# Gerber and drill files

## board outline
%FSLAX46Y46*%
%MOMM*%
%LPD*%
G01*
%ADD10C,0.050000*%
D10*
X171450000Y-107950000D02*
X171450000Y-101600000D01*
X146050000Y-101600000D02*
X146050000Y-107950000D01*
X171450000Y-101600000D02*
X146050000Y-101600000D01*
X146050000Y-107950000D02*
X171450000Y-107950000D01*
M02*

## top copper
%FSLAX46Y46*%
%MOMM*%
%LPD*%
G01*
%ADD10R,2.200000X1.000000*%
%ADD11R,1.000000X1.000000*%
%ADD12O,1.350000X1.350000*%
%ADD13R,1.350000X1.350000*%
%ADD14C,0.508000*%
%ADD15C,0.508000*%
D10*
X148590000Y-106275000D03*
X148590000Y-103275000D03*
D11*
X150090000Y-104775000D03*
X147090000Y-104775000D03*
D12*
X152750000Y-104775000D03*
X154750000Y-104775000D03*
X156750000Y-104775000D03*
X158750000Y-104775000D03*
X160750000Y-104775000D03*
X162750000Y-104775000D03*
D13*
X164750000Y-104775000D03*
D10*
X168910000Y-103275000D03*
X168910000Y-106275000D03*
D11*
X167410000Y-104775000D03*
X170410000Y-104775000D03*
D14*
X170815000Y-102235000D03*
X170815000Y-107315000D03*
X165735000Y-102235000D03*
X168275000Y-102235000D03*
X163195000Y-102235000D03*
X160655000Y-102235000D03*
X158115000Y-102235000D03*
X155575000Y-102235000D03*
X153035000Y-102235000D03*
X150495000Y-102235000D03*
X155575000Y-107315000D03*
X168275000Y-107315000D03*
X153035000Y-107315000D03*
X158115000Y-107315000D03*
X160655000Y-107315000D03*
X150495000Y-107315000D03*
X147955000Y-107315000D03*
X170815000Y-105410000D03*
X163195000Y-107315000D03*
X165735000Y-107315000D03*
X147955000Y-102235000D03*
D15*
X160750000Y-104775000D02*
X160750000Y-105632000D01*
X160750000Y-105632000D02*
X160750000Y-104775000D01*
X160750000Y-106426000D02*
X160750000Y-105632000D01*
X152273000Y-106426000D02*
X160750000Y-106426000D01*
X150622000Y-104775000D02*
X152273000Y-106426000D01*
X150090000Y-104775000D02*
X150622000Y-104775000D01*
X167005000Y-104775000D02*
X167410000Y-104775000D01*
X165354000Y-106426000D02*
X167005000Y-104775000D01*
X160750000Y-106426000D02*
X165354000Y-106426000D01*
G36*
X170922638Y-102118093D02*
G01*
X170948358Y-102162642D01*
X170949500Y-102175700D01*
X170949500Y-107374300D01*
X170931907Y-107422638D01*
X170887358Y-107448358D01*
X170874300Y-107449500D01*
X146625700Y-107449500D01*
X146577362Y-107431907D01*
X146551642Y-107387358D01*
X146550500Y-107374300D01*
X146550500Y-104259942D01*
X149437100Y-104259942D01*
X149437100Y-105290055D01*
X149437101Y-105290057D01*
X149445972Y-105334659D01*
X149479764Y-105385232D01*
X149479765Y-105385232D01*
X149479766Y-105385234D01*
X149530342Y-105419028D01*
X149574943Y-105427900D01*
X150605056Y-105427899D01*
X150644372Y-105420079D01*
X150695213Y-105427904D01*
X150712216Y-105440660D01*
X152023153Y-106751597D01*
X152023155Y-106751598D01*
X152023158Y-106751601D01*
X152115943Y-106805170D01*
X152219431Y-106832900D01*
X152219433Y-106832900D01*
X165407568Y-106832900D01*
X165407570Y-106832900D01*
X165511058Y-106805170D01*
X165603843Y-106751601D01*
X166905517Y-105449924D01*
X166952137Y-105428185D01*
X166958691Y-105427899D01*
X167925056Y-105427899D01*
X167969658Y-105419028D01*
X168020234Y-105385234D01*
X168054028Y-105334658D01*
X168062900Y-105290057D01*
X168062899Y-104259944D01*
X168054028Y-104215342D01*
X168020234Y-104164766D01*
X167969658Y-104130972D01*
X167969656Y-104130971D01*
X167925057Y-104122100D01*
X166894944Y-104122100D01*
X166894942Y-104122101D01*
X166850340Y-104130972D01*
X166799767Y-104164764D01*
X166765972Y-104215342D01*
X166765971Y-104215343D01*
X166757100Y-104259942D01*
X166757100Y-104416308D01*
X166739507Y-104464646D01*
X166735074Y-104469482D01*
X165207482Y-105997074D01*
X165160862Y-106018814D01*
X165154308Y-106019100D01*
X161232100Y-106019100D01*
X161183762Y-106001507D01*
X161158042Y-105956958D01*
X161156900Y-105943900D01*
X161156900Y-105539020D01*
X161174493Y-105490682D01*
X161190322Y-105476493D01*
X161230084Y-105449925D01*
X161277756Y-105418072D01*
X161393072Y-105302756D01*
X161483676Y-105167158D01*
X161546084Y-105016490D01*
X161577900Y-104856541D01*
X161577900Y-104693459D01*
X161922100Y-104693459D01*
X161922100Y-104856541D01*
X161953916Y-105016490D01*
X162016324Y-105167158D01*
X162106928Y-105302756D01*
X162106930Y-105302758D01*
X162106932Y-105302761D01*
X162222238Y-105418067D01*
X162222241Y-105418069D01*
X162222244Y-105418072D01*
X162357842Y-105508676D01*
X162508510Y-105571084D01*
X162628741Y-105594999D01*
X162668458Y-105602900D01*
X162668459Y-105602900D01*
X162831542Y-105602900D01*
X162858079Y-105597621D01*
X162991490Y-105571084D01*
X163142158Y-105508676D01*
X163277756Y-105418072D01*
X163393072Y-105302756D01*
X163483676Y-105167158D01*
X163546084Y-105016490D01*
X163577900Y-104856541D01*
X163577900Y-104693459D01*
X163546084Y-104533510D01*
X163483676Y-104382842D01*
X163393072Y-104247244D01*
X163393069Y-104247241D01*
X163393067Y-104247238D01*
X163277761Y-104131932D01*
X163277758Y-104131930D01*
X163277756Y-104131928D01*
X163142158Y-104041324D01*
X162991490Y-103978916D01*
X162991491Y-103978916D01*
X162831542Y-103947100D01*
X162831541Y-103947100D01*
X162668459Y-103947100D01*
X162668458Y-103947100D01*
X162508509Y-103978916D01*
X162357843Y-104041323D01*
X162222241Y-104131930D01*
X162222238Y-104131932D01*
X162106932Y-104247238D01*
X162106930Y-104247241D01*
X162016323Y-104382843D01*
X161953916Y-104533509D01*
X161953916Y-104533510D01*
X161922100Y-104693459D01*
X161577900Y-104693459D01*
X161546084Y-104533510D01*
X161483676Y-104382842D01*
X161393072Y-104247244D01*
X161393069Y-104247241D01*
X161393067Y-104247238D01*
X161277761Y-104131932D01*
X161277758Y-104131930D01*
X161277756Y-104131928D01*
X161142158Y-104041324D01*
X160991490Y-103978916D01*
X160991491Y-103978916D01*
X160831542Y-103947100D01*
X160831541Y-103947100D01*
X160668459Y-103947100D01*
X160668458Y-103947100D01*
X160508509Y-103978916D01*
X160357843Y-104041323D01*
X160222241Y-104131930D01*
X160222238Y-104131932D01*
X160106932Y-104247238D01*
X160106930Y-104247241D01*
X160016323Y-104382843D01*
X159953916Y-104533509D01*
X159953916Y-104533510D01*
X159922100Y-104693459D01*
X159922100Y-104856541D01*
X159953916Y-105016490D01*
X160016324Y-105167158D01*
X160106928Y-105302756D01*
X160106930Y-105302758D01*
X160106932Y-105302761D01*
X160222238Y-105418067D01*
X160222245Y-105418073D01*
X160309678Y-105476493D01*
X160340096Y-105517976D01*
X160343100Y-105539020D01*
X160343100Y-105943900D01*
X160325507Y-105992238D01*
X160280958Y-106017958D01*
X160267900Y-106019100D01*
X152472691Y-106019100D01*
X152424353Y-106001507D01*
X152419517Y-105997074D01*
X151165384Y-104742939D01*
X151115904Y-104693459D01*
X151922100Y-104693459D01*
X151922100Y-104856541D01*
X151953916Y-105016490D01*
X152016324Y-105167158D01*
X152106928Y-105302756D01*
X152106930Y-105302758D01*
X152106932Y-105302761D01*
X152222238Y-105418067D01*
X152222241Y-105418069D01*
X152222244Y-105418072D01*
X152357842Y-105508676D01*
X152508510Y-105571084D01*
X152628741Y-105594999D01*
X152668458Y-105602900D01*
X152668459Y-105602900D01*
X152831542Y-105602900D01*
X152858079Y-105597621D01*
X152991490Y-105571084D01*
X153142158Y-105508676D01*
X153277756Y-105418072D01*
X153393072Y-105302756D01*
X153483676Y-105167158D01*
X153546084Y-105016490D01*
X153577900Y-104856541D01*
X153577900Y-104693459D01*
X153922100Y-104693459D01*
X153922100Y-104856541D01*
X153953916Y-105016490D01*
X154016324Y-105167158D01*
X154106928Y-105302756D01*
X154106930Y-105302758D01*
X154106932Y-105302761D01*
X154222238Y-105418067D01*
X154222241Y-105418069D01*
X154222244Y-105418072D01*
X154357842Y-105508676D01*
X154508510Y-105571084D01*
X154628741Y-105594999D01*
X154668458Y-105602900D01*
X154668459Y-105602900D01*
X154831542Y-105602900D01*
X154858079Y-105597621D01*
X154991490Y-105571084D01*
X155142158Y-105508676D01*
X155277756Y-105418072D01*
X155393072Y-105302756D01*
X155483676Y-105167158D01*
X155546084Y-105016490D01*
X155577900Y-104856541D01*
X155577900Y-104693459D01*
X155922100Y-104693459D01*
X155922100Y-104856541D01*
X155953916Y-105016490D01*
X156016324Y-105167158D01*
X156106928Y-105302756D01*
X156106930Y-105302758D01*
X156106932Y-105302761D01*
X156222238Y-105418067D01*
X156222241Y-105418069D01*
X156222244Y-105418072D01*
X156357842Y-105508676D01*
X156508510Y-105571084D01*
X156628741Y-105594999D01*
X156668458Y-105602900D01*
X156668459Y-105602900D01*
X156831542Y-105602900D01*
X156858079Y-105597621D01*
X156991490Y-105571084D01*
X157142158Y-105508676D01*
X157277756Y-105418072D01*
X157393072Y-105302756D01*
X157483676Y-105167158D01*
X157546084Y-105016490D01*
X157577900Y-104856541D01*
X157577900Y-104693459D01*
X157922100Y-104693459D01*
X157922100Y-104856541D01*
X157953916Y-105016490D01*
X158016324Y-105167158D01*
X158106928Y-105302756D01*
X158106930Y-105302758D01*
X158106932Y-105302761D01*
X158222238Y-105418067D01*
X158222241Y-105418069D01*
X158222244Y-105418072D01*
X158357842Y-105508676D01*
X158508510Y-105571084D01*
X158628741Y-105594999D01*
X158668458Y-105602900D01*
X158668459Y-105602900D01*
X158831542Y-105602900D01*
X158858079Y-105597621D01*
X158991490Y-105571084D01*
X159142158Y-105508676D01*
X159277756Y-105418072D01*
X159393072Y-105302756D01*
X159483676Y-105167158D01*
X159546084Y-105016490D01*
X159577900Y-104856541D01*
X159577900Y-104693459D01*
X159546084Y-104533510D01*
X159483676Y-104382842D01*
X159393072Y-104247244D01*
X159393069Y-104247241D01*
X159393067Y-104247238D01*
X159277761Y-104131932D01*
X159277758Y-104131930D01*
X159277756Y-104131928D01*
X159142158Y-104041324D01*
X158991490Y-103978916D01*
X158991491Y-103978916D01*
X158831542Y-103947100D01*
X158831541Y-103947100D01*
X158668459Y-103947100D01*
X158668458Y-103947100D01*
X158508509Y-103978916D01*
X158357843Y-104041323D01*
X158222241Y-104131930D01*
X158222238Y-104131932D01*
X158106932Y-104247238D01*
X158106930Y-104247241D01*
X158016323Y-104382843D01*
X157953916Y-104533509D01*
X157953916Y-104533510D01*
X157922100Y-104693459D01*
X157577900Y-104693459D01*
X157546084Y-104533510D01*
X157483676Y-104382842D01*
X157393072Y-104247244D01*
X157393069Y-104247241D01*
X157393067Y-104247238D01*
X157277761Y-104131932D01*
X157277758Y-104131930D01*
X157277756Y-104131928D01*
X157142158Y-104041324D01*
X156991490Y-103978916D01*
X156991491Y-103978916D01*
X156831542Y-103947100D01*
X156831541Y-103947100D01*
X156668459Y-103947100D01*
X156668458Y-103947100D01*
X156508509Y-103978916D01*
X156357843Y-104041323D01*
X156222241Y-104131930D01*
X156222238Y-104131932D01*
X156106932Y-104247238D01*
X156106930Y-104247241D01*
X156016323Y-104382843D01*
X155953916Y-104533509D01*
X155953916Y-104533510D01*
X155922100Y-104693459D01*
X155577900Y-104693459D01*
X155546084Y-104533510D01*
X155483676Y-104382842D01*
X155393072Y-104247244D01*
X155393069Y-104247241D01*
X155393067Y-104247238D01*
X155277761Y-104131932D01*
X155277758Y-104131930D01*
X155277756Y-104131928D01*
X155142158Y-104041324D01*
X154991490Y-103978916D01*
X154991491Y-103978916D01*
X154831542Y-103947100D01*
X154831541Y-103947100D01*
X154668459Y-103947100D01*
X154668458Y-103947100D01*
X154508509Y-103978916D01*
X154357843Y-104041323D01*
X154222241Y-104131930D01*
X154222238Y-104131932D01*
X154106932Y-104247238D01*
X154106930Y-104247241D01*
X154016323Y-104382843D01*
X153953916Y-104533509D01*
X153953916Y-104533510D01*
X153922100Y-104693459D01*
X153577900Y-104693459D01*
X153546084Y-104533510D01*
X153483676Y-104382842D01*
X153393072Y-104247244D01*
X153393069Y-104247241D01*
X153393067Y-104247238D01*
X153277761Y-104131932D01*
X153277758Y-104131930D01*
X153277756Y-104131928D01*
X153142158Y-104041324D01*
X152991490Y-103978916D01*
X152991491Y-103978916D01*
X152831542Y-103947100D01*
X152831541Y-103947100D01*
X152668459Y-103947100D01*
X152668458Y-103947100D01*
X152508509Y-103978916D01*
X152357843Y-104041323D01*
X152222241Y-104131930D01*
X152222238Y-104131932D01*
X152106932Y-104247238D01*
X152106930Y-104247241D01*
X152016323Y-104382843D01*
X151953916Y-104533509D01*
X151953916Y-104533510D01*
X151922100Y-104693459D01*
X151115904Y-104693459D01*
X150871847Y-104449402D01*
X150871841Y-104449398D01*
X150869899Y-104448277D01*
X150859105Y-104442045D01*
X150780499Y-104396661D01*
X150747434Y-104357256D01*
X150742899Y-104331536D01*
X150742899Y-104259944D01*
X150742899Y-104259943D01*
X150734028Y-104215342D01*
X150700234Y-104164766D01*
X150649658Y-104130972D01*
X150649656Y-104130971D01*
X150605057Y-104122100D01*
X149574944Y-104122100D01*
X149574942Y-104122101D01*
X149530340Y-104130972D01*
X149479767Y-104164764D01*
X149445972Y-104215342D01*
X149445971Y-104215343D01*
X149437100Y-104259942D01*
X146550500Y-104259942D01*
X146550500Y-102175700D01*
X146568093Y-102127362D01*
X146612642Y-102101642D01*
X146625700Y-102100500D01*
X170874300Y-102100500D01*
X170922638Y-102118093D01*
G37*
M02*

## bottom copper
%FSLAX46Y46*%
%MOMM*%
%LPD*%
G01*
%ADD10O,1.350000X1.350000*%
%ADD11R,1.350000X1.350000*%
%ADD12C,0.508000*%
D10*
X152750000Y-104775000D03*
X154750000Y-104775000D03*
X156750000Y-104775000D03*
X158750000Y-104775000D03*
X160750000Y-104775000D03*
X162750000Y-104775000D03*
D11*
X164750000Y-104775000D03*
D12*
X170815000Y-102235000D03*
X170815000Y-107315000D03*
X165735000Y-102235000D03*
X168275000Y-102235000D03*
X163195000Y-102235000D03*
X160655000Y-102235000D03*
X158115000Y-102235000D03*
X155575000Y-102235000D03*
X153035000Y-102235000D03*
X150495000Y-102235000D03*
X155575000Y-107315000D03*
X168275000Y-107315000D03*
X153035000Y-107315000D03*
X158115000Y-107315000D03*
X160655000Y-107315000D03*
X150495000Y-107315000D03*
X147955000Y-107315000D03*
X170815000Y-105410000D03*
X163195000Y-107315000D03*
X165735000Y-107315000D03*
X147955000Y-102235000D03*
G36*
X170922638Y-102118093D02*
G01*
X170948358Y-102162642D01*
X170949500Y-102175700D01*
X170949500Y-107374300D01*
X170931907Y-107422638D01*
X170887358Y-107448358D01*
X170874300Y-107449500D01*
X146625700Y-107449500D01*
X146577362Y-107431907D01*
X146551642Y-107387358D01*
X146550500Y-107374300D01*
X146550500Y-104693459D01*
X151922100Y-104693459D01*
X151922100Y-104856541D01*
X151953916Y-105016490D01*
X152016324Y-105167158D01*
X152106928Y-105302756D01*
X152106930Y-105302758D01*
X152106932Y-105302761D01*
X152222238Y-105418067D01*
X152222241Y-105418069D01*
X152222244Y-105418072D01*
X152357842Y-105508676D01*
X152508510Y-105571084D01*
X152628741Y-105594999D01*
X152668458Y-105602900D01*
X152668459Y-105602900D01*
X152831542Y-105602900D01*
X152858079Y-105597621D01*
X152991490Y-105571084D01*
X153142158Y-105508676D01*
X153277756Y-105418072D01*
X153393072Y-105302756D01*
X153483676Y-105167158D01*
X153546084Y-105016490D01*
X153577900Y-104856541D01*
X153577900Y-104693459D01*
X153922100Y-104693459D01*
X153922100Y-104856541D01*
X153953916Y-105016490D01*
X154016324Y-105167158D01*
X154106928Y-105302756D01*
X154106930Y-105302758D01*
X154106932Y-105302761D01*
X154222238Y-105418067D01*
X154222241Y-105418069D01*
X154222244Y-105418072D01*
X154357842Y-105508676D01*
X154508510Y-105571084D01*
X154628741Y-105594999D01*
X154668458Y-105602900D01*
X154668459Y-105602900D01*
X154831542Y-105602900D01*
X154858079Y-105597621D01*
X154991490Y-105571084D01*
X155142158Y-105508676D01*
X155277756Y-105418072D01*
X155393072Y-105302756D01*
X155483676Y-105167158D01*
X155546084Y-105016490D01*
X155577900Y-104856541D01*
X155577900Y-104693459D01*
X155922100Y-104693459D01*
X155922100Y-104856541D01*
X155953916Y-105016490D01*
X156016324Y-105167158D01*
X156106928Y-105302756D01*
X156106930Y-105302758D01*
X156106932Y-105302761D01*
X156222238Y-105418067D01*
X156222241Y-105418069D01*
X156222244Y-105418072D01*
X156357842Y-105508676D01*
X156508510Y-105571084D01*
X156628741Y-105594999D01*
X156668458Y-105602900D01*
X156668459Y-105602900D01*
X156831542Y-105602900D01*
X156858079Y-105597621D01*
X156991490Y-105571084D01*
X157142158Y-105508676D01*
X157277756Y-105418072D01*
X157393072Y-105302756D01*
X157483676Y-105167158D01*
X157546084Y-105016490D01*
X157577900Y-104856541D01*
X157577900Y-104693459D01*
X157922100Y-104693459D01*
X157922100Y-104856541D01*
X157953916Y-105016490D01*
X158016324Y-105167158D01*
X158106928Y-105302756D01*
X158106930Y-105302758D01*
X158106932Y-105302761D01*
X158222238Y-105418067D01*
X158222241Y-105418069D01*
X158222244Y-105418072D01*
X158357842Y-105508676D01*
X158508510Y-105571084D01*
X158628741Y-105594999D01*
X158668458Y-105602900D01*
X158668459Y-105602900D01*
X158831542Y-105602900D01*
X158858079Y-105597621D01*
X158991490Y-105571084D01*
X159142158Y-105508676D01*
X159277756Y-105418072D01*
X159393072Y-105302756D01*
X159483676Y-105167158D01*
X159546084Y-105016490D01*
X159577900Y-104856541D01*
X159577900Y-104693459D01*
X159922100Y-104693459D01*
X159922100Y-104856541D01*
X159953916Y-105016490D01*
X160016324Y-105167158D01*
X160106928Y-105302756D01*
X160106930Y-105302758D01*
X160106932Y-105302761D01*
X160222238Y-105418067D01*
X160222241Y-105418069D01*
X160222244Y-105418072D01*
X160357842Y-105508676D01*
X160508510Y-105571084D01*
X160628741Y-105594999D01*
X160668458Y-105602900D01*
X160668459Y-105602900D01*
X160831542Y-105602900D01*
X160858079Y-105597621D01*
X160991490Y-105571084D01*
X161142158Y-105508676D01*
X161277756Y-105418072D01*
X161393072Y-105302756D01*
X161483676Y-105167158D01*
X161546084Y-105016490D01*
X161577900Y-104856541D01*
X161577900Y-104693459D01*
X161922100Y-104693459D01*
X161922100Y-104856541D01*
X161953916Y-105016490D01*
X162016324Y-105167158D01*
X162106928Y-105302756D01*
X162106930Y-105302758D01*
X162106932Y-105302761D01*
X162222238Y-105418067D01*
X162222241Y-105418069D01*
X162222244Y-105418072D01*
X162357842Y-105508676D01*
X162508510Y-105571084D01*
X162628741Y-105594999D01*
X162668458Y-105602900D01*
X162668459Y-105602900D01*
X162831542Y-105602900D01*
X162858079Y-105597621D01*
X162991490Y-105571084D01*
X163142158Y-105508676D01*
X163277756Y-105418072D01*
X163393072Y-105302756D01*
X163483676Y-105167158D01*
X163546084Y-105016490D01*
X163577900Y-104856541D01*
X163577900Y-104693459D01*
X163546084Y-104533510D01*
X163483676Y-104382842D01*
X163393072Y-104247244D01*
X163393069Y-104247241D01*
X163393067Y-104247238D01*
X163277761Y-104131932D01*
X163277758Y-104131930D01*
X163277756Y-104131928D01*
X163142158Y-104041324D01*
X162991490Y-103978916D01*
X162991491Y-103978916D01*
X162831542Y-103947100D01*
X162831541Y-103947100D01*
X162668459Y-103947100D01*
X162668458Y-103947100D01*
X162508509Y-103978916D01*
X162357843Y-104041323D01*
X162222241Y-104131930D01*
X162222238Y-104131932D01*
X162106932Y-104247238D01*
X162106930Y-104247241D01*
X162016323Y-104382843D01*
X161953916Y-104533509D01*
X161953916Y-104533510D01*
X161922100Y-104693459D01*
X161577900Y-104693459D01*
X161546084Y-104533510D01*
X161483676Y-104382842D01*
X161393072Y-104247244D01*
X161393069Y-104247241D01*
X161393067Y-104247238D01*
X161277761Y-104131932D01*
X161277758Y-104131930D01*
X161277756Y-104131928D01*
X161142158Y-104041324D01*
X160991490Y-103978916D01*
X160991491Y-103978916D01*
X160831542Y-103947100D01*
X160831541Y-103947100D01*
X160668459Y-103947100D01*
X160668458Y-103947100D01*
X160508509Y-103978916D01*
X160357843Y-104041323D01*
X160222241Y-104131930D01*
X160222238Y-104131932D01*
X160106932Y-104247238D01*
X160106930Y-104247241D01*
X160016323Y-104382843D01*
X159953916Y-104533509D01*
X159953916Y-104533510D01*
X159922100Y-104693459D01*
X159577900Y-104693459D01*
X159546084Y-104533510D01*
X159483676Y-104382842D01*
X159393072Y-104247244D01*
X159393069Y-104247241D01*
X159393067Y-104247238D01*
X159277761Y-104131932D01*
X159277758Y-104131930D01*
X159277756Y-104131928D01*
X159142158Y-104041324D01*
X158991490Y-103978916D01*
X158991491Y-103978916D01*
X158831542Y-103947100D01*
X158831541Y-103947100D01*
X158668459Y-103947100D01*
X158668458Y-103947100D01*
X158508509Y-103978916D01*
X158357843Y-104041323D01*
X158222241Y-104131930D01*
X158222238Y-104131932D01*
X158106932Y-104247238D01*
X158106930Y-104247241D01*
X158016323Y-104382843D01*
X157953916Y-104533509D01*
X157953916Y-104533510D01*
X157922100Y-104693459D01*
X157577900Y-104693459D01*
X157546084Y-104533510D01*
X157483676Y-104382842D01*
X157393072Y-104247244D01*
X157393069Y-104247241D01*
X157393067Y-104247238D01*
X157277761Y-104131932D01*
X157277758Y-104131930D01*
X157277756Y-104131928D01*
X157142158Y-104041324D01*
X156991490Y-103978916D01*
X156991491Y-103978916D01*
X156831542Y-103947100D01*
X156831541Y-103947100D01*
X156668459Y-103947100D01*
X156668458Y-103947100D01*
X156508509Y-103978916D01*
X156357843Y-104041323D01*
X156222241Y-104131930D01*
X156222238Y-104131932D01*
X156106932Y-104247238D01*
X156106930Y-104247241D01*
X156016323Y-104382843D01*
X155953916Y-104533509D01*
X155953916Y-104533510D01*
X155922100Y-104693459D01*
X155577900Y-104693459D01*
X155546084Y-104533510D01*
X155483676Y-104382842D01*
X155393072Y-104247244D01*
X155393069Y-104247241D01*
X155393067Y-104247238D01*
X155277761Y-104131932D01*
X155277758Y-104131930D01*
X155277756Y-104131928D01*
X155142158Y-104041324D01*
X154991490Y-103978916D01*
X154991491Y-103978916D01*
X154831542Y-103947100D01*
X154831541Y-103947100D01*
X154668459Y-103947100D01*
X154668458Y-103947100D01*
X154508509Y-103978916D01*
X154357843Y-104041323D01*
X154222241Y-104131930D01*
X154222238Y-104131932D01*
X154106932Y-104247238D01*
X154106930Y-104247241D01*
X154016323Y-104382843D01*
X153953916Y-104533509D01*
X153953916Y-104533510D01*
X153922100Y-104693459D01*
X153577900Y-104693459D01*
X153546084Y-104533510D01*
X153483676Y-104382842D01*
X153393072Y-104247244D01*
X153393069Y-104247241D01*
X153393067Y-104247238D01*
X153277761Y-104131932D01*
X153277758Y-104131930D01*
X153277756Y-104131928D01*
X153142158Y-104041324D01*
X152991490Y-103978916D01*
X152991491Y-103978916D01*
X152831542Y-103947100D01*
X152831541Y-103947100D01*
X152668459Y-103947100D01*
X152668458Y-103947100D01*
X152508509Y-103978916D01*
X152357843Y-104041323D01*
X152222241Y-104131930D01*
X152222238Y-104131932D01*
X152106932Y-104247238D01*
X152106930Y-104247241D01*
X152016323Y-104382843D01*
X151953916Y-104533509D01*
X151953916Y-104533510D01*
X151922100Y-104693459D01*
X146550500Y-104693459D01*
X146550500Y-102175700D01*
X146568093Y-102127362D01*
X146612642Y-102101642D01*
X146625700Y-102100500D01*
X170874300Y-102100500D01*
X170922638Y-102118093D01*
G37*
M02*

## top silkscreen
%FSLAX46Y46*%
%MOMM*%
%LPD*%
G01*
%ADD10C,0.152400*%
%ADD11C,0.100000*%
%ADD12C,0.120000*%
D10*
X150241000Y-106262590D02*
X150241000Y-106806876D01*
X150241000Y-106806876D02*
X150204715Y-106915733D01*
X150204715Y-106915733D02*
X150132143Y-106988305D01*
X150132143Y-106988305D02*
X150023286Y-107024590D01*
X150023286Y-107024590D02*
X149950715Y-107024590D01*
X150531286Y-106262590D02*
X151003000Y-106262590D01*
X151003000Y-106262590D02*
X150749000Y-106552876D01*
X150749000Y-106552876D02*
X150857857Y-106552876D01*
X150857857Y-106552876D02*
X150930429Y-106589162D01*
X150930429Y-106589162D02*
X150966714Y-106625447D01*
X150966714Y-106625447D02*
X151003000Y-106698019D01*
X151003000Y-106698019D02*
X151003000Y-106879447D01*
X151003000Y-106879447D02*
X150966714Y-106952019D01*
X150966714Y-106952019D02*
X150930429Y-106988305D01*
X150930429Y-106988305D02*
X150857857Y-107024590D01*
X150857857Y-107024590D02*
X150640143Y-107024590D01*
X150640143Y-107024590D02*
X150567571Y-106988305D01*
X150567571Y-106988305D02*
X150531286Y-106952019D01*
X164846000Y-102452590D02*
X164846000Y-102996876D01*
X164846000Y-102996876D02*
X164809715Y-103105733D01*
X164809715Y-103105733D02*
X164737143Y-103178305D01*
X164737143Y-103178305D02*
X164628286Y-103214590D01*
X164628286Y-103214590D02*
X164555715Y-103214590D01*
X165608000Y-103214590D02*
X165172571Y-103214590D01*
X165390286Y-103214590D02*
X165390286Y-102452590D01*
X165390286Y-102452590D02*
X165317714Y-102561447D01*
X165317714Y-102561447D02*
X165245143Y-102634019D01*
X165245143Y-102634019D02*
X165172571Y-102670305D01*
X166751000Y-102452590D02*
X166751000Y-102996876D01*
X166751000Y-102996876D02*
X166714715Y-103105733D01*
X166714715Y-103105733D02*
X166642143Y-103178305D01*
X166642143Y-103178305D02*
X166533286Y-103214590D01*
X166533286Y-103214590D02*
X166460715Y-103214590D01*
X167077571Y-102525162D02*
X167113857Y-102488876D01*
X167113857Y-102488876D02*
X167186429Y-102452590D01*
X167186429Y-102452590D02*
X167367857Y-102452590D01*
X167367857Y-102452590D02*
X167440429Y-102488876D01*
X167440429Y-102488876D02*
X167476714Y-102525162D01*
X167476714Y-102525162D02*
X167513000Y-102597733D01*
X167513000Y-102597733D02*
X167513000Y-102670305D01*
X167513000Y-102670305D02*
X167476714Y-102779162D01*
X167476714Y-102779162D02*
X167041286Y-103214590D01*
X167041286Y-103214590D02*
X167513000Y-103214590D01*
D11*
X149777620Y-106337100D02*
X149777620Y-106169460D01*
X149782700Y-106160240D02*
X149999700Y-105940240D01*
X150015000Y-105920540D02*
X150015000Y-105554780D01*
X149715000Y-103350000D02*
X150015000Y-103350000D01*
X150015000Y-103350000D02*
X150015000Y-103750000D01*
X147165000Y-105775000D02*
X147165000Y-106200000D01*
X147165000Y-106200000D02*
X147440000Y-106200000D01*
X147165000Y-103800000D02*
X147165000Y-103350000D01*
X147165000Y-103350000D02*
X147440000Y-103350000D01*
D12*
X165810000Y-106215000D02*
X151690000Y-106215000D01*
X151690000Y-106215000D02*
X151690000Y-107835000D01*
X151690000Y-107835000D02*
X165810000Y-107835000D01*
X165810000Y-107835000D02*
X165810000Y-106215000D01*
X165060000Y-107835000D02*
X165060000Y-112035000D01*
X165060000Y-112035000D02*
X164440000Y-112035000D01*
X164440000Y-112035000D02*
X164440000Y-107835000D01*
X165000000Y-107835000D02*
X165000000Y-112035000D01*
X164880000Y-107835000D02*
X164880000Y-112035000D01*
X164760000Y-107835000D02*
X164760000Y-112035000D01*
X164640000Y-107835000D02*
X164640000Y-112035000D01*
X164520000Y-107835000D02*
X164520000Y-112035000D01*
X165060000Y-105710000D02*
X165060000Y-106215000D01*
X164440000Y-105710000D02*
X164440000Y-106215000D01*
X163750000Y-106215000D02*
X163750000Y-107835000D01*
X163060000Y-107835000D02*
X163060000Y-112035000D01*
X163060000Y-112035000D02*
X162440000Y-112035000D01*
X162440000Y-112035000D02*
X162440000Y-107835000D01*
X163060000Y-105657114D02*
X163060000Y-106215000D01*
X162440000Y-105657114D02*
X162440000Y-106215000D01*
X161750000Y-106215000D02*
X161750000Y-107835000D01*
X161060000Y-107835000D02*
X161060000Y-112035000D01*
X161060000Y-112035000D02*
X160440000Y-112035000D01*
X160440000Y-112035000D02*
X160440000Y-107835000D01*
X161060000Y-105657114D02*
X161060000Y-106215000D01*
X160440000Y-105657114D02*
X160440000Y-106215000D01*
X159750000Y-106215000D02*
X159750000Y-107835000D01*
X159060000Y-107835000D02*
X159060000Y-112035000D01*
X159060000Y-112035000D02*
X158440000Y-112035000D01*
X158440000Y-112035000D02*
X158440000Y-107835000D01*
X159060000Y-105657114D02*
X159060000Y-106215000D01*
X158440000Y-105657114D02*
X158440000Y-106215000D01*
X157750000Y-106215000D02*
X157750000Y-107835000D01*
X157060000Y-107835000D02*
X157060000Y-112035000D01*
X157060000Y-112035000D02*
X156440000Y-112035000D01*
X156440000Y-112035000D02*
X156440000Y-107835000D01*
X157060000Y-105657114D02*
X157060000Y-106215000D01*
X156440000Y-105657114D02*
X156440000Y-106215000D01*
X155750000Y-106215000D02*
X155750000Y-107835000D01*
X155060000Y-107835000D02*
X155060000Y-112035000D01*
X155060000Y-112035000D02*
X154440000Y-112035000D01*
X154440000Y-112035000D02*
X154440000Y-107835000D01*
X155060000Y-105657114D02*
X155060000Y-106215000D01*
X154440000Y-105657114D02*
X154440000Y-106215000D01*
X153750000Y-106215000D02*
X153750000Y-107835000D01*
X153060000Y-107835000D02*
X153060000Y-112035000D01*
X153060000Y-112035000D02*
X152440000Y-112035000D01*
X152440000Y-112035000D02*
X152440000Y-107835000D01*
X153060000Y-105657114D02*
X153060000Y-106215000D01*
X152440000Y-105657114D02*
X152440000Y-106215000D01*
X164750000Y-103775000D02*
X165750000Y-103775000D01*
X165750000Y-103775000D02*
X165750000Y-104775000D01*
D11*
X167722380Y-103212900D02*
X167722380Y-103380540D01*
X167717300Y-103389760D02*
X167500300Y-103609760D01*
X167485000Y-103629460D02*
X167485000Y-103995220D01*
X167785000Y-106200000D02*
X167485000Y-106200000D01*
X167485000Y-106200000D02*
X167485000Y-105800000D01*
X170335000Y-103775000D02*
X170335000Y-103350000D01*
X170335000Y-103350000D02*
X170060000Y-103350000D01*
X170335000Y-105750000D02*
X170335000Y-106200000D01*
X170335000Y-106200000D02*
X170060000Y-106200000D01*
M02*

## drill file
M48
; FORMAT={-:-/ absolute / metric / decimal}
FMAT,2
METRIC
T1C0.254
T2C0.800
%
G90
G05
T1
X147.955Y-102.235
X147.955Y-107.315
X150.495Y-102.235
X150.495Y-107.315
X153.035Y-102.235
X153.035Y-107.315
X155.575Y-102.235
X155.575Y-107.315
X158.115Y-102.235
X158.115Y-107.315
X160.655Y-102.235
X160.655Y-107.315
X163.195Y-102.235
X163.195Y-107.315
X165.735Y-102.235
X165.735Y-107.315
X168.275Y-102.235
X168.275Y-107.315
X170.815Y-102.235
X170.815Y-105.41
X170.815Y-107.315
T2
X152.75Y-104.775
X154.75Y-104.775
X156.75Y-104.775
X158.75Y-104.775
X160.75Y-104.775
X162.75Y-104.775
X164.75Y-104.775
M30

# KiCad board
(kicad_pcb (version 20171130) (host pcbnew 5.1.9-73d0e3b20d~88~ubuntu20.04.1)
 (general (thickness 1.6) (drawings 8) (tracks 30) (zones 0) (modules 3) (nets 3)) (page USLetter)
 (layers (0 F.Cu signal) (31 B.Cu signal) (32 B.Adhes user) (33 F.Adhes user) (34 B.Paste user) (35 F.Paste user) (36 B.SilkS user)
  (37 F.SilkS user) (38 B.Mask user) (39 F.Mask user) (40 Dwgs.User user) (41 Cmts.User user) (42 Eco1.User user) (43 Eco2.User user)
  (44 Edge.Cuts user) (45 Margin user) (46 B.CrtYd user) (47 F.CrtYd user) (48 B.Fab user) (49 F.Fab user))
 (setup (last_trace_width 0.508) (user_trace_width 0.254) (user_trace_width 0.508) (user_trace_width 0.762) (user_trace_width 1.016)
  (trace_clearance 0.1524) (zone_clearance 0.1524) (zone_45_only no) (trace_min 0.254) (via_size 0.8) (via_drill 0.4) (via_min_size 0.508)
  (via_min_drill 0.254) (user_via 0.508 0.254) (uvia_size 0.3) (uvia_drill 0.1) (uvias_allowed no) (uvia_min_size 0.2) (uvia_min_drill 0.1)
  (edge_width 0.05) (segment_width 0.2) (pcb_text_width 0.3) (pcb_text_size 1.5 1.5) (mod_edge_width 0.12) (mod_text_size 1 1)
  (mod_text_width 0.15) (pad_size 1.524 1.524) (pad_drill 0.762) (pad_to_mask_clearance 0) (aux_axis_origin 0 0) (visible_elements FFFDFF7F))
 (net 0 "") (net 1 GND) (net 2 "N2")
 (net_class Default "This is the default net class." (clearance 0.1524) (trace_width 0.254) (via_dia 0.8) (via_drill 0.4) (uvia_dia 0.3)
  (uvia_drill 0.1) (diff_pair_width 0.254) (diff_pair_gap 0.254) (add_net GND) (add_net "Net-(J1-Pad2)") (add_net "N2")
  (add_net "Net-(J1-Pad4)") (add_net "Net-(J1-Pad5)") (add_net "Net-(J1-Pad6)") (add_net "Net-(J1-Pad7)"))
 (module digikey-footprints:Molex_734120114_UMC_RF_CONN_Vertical (layer F.Cu) (at 148.59 104.775 90)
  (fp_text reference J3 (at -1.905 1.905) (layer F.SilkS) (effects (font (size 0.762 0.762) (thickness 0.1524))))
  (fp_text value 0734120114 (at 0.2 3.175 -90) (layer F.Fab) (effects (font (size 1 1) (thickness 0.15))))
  (fp_line (start -1.5621 1.18762) (end -1.39446 1.18762) (layer F.SilkS) (width 0.1))
  (fp_line (start -1.38524 1.1927) (end -1.16524 1.4097) (layer F.SilkS) (width 0.1))
  (fp_line (start -1.14554 1.425) (end -0.77978 1.425) (layer F.SilkS) (width 0.1))
  (fp_line (start 1.425 1.125) (end 1.425 1.425) (layer F.SilkS) (width 0.1))
  (fp_line (start 1.425 1.425) (end 1.025 1.425) (layer F.SilkS) (width 0.1))
  (fp_line (start -1 -1.425) (end -1.425 -1.425) (layer F.SilkS) (width 0.1))
  (fp_line (start -1.425 -1.425) (end -1.425 -1.15) (layer F.SilkS) (width 0.1))
  (fp_line (start 0.975 -1.425) (end 1.425 -1.425) (layer F.SilkS) (width 0.1))
  (fp_line (start 1.425 -1.425) (end 1.425 -1.15) (layer F.SilkS) (width 0.1))
  (pad 1 smd rect (at -1.5 0 90) (size 1 2.2) (layers F.Cu F.Paste F.Mask) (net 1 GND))
  (pad 1 smd rect (at 1.5 0 90) (size 1 2.2) (layers F.Cu F.Paste F.Mask) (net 1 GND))
  (pad 2 smd rect (at 0 1.5 90) (size 1 1) (layers F.Cu F.Paste F.Mask) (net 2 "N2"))
  (pad 1 smd rect (at 0 -1.5 90) (size 1 1) (layers F.Cu F.Paste F.Mask) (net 1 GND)))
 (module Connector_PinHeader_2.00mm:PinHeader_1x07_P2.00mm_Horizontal (layer F.Cu) (at 164.75 104.775 270)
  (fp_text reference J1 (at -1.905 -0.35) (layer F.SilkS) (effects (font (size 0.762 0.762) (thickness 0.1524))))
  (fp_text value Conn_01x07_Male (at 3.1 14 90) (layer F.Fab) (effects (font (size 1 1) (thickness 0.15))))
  (fp_line (start 1.44 -1.06) (end 1.44 13.06) (layer F.SilkS) (width 0.12))
  (fp_line (start 1.44 13.06) (end 3.06 13.06) (layer F.SilkS) (width 0.12))
  (fp_line (start 3.06 13.06) (end 3.06 -1.06) (layer F.SilkS) (width 0.12))
  (fp_line (start 3.06 -1.06) (end 1.44 -1.06) (layer F.SilkS) (width 0.12))
  (fp_line (start 3.06 -0.31) (end 7.26 -0.31) (layer F.SilkS) (width 0.12))
  (fp_line (start 7.26 -0.31) (end 7.26 0.31) (layer F.SilkS) (width 0.12))
  (fp_line (start 7.26 0.31) (end 3.06 0.31) (layer F.SilkS) (width 0.12))
  (fp_line (start 3.06 -0.25) (end 7.26 -0.25) (layer F.SilkS) (width 0.12))
  (fp_line (start 3.06 -0.13) (end 7.26 -0.13) (layer F.SilkS) (width 0.12))
  (fp_line (start 3.06 -0.01) (end 7.26 -0.01) (layer F.SilkS) (width 0.12))
  (fp_line (start 3.06 0.11) (end 7.26 0.11) (layer F.SilkS) (width 0.12))
  (fp_line (start 3.06 0.23) (end 7.26 0.23) (layer F.SilkS) (width 0.12))
  (fp_line (start 0.935 -0.31) (end 1.44 -0.31) (layer F.SilkS) (width 0.12))
  (fp_line (start 0.935 0.31) (end 1.44 0.31) (layer F.SilkS) (width 0.12))
  (fp_line (start 1.44 1) (end 3.06 1) (layer F.SilkS) (width 0.12))
  (fp_line (start 3.06 1.69) (end 7.26 1.69) (layer F.SilkS) (width 0.12))
  (fp_line (start 7.26 1.69) (end 7.26 2.31) (layer F.SilkS) (width 0.12))
  (fp_line (start 7.26 2.31) (end 3.06 2.31) (layer F.SilkS) (width 0.12))
  (fp_line (start 0.882114 1.69) (end 1.44 1.69) (layer F.SilkS) (width 0.12))
  (fp_line (start 0.882114 2.31) (end 1.44 2.31) (layer F.SilkS) (width 0.12))
  (fp_line (start 1.44 3) (end 3.06 3) (layer F.SilkS) (width 0.12))
  (fp_line (start 3.06 3.69) (end 7.26 3.69) (layer F.SilkS) (width 0.12))
  (fp_line (start 7.26 3.69) (end 7.26 4.31) (layer F.SilkS) (width 0.12))
  (fp_line (start 7.26 4.31) (end 3.06 4.31) (layer F.SilkS) (width 0.12))
  (fp_line (start 0.882114 3.69) (end 1.44 3.69) (layer F.SilkS) (width 0.12))
  (fp_line (start 0.882114 4.31) (end 1.44 4.31) (layer F.SilkS) (width 0.12))
  (fp_line (start 1.44 5) (end 3.06 5) (layer F.SilkS) (width 0.12))
  (fp_line (start 3.06 5.69) (end 7.26 5.69) (layer F.SilkS) (width 0.12))
  (fp_line (start 7.26 5.69) (end 7.26 6.31) (layer F.SilkS) (width 0.12))
  (fp_line (start 7.26 6.31) (end 3.06 6.31) (layer F.SilkS) (width 0.12))
  (fp_line (start 0.882114 5.69) (end 1.44 5.69) (layer F.SilkS) (width 0.12))
  (fp_line (start 0.882114 6.31) (end 1.44 6.31) (layer F.SilkS) (width 0.12))
  (fp_line (start 1.44 7) (end 3.06 7) (layer F.SilkS) (width 0.12))
  (fp_line (start 3.06 7.69) (end 7.26 7.69) (layer F.SilkS) (width 0.12))
  (fp_line (start 7.26 7.69) (end 7.26 8.31) (layer F.SilkS) (width 0.12))
  (fp_line (start 7.26 8.31) (end 3.06 8.31) (layer F.SilkS) (width 0.12))
  (fp_line (start 0.882114 7.69) (end 1.44 7.69) (layer F.SilkS) (width 0.12))
  (fp_line (start 0.882114 8.31) (end 1.44 8.31) (layer F.SilkS) (width 0.12))
  (fp_line (start 1.44 9) (end 3.06 9) (layer F.SilkS) (width 0.12))
  (fp_line (start 3.06 9.69) (end 7.26 9.69) (layer F.SilkS) (width 0.12))
  (fp_line (start 7.26 9.69) (end 7.26 10.31) (layer F.SilkS) (width 0.12))
  (fp_line (start 7.26 10.31) (end 3.06 10.31) (layer F.SilkS) (width 0.12))
  (fp_line (start 0.882114 9.69) (end 1.44 9.69) (layer F.SilkS) (width 0.12))
  (fp_line (start 0.882114 10.31) (end 1.44 10.31) (layer F.SilkS) (width 0.12))
  (fp_line (start 1.44 11) (end 3.06 11) (layer F.SilkS) (width 0.12))
  (fp_line (start 3.06 11.69) (end 7.26 11.69) (layer F.SilkS) (width 0.12))
  (fp_line (start 7.26 11.69) (end 7.26 12.31) (layer F.SilkS) (width 0.12))
  (fp_line (start 7.26 12.31) (end 3.06 12.31) (layer F.SilkS) (width 0.12))
  (fp_line (start 0.882114 11.69) (end 1.44 11.69) (layer F.SilkS) (width 0.12))
  (fp_line (start 0.882114 12.31) (end 1.44 12.31) (layer F.SilkS) (width 0.12))
  (fp_line (start -1 0) (end -1 -1) (layer F.SilkS) (width 0.12))
  (fp_line (start -1 -1) (end 0 -1) (layer F.SilkS) (width 0.12))
  (pad 7 thru_hole oval (at 0 12 270) (size 1.35 1.35) (drill 0.8) (layers *.Cu *.Mask))
  (pad 6 thru_hole oval (at 0 10 270) (size 1.35 1.35) (drill 0.8) (layers *.Cu *.Mask))
  (pad 5 thru_hole oval (at 0 8 270) (size 1.35 1.35) (drill 0.8) (layers *.Cu *.Mask))
  (pad 4 thru_hole oval (at 0 6 270) (size 1.35 1.35) (drill 0.8) (layers *.Cu *.Mask))
  (pad 3 thru_hole oval (at 0 4 270) (size 1.35 1.35) (drill 0.8) (layers *.Cu *.Mask) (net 2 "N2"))
  (pad 2 thru_hole oval (at 0 2 270) (size 1.35 1.35) (drill 0.8) (layers *.Cu *.Mask))
  (pad 1 thru_hole rect (at 0 0 270) (size 1.35 1.35) (drill 0.8) (layers *.Cu *.Mask) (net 1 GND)))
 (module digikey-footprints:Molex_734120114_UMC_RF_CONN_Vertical (layer F.Cu) (at 168.91 104.775 270)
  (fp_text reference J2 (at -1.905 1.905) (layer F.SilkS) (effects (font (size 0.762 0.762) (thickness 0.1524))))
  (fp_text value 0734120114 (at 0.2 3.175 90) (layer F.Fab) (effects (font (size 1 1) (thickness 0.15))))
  (fp_line (start -1.5621 1.18762) (end -1.39446 1.18762) (layer F.SilkS) (width 0.1))
  (fp_line (start -1.38524 1.1927) (end -1.16524 1.4097) (layer F.SilkS) (width 0.1))
  (fp_line (start -1.14554 1.425) (end -0.77978 1.425) (layer F.SilkS) (width 0.1))
  (fp_line (start 1.425 1.125) (end 1.425 1.425) (layer F.SilkS) (width 0.1))
  (fp_line (start 1.425 1.425) (end 1.025 1.425) (layer F.SilkS) (width 0.1))
  (fp_line (start -1 -1.425) (end -1.425 -1.425) (layer F.SilkS) (width 0.1))
  (fp_line (start -1.425 -1.425) (end -1.425 -1.15) (layer F.SilkS) (width 0.1))
  (fp_line (start 0.975 -1.425) (end 1.425 -1.425) (layer F.SilkS) (width 0.1))
  (fp_line (start 1.425 -1.425) (end 1.425 -1.15) (layer F.SilkS) (width 0.1))
  (pad 1 smd rect (at -1.5 0 270) (size 1 2.2) (layers F.Cu F.Paste F.Mask) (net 1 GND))
  (pad 1 smd rect (at 1.5 0 270) (size 1 2.2) (layers F.Cu F.Paste F.Mask) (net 1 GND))
  (pad 2 smd rect (at 0 1.5 270) (size 1 1) (layers F.Cu F.Paste F.Mask) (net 2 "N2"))
  (pad 1 smd rect (at 0 -1.5 270) (size 1 1) (layers F.Cu F.Paste F.Mask) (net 1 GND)))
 (gr_line (start 171.45 107.95) (end 171.45 101.6) (layer Edge.Cuts) (width 0.05))
 (gr_line (start 146.05 101.6) (end 146.05 107.95) (layer Edge.Cuts) (width 0.05))
 (gr_line (start 171.45 101.6) (end 146.05 101.6) (layer Edge.Cuts) (width 0.05))
 (gr_line (start 146.05 107.95) (end 171.45 107.95) (layer Edge.Cuts) (width 0.05))
 (segment (start 160.75 104.775) (end 160.75 105.632) (width 0.508) (layer F.Cu) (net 2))
 (segment (start 160.75 105.632) (end 160.75 104.775) (width 0.508) (layer F.Cu) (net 2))
 (segment (start 160.75 106.426) (end 160.75 105.632) (width 0.508) (layer F.Cu) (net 2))
 (segment (start 152.273 106.426) (end 160.75 106.426) (width 0.508) (layer F.Cu) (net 2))
 (segment (start 150.622 104.775) (end 152.273 106.426) (width 0.508) (layer F.Cu) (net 2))
 (segment (start 150.09 104.775) (end 150.622 104.775) (width 0.508) (layer F.Cu) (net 2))
 (segment (start 167.005 104.775) (end 167.41 104.775) (width 0.508) (layer F.Cu) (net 2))
 (segment (start 165.354 106.426) (end 167.005 104.775) (width 0.508) (layer F.Cu) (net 2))
 (segment (start 160.75 106.426) (end 165.354 106.426) (width 0.508) (layer F.Cu) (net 2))
 (via (at 170.815 102.235) (size 0.508) (drill 0.254) (layers F.Cu B.Cu) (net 1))
 (via (at 170.815 107.315) (size 0.508) (drill 0.254) (layers F.Cu B.Cu) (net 1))
 (via (at 165.735 102.235) (size 0.508) (drill 0.254) (layers F.Cu B.Cu) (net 1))
 (via (at 168.275 102.235) (size 0.508) (drill 0.254) (layers F.Cu B.Cu) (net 1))
 (via (at 163.195 102.235) (size 0.508) (drill 0.254) (layers F.Cu B.Cu) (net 1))
 (via (at 160.655 102.235) (size 0.508) (drill 0.254) (layers F.Cu B.Cu) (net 1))
 (via (at 158.115 102.235) (size 0.508) (drill 0.254) (layers F.Cu B.Cu) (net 1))
 (via (at 155.575 102.235) (size 0.508) (drill 0.254) (layers F.Cu B.Cu) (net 1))
 (via (at 153.035 102.235) (size 0.508) (drill 0.254) (layers F.Cu B.Cu) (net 1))
 (via (at 150.495 102.235) (size 0.508) (drill 0.254) (layers F.Cu B.Cu) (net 1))
 (via (at 155.575 107.315) (size 0.508) (drill 0.254) (layers F.Cu B.Cu) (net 1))
 (via (at 168.275 107.315) (size 0.508) (drill 0.254) (layers F.Cu B.Cu) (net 1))
 (via (at 153.035 107.315) (size 0.508) (drill 0.254) (layers F.Cu B.Cu) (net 1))
 (via (at 158.115 107.315) (size 0.508) (drill 0.254) (layers F.Cu B.Cu) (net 1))
 (via (at 160.655 107.315) (size 0.508) (drill 0.254) (layers F.Cu B.Cu) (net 1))
 (via (at 150.495 107.315) (size 0.508) (drill 0.254) (layers F.Cu B.Cu) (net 1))
 (via (at 147.955 107.315) (size 0.508) (drill 0.254) (layers F.Cu B.Cu) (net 1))
 (via (at 170.815 105.41) (size 0.508) (drill 0.254) (layers F.Cu B.Cu) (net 1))
 (via (at 163.195 107.315) (size 0.508) (drill 0.254) (layers F.Cu B.Cu) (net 1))
 (via (at 165.735 107.315) (size 0.508) (drill 0.254) (layers F.Cu B.Cu) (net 1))
 (via (at 147.955 102.235) (size 0.508) (drill 0.254) (layers F.Cu B.Cu) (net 1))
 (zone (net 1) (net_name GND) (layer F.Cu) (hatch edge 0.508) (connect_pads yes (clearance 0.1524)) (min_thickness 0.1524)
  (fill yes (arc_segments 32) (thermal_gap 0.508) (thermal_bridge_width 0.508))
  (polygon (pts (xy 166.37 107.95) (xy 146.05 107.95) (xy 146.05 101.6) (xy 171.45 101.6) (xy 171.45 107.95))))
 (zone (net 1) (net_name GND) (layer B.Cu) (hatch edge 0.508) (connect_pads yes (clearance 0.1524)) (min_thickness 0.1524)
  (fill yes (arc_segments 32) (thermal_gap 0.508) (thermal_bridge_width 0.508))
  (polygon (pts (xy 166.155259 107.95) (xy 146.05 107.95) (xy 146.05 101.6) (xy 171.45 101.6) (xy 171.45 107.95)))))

